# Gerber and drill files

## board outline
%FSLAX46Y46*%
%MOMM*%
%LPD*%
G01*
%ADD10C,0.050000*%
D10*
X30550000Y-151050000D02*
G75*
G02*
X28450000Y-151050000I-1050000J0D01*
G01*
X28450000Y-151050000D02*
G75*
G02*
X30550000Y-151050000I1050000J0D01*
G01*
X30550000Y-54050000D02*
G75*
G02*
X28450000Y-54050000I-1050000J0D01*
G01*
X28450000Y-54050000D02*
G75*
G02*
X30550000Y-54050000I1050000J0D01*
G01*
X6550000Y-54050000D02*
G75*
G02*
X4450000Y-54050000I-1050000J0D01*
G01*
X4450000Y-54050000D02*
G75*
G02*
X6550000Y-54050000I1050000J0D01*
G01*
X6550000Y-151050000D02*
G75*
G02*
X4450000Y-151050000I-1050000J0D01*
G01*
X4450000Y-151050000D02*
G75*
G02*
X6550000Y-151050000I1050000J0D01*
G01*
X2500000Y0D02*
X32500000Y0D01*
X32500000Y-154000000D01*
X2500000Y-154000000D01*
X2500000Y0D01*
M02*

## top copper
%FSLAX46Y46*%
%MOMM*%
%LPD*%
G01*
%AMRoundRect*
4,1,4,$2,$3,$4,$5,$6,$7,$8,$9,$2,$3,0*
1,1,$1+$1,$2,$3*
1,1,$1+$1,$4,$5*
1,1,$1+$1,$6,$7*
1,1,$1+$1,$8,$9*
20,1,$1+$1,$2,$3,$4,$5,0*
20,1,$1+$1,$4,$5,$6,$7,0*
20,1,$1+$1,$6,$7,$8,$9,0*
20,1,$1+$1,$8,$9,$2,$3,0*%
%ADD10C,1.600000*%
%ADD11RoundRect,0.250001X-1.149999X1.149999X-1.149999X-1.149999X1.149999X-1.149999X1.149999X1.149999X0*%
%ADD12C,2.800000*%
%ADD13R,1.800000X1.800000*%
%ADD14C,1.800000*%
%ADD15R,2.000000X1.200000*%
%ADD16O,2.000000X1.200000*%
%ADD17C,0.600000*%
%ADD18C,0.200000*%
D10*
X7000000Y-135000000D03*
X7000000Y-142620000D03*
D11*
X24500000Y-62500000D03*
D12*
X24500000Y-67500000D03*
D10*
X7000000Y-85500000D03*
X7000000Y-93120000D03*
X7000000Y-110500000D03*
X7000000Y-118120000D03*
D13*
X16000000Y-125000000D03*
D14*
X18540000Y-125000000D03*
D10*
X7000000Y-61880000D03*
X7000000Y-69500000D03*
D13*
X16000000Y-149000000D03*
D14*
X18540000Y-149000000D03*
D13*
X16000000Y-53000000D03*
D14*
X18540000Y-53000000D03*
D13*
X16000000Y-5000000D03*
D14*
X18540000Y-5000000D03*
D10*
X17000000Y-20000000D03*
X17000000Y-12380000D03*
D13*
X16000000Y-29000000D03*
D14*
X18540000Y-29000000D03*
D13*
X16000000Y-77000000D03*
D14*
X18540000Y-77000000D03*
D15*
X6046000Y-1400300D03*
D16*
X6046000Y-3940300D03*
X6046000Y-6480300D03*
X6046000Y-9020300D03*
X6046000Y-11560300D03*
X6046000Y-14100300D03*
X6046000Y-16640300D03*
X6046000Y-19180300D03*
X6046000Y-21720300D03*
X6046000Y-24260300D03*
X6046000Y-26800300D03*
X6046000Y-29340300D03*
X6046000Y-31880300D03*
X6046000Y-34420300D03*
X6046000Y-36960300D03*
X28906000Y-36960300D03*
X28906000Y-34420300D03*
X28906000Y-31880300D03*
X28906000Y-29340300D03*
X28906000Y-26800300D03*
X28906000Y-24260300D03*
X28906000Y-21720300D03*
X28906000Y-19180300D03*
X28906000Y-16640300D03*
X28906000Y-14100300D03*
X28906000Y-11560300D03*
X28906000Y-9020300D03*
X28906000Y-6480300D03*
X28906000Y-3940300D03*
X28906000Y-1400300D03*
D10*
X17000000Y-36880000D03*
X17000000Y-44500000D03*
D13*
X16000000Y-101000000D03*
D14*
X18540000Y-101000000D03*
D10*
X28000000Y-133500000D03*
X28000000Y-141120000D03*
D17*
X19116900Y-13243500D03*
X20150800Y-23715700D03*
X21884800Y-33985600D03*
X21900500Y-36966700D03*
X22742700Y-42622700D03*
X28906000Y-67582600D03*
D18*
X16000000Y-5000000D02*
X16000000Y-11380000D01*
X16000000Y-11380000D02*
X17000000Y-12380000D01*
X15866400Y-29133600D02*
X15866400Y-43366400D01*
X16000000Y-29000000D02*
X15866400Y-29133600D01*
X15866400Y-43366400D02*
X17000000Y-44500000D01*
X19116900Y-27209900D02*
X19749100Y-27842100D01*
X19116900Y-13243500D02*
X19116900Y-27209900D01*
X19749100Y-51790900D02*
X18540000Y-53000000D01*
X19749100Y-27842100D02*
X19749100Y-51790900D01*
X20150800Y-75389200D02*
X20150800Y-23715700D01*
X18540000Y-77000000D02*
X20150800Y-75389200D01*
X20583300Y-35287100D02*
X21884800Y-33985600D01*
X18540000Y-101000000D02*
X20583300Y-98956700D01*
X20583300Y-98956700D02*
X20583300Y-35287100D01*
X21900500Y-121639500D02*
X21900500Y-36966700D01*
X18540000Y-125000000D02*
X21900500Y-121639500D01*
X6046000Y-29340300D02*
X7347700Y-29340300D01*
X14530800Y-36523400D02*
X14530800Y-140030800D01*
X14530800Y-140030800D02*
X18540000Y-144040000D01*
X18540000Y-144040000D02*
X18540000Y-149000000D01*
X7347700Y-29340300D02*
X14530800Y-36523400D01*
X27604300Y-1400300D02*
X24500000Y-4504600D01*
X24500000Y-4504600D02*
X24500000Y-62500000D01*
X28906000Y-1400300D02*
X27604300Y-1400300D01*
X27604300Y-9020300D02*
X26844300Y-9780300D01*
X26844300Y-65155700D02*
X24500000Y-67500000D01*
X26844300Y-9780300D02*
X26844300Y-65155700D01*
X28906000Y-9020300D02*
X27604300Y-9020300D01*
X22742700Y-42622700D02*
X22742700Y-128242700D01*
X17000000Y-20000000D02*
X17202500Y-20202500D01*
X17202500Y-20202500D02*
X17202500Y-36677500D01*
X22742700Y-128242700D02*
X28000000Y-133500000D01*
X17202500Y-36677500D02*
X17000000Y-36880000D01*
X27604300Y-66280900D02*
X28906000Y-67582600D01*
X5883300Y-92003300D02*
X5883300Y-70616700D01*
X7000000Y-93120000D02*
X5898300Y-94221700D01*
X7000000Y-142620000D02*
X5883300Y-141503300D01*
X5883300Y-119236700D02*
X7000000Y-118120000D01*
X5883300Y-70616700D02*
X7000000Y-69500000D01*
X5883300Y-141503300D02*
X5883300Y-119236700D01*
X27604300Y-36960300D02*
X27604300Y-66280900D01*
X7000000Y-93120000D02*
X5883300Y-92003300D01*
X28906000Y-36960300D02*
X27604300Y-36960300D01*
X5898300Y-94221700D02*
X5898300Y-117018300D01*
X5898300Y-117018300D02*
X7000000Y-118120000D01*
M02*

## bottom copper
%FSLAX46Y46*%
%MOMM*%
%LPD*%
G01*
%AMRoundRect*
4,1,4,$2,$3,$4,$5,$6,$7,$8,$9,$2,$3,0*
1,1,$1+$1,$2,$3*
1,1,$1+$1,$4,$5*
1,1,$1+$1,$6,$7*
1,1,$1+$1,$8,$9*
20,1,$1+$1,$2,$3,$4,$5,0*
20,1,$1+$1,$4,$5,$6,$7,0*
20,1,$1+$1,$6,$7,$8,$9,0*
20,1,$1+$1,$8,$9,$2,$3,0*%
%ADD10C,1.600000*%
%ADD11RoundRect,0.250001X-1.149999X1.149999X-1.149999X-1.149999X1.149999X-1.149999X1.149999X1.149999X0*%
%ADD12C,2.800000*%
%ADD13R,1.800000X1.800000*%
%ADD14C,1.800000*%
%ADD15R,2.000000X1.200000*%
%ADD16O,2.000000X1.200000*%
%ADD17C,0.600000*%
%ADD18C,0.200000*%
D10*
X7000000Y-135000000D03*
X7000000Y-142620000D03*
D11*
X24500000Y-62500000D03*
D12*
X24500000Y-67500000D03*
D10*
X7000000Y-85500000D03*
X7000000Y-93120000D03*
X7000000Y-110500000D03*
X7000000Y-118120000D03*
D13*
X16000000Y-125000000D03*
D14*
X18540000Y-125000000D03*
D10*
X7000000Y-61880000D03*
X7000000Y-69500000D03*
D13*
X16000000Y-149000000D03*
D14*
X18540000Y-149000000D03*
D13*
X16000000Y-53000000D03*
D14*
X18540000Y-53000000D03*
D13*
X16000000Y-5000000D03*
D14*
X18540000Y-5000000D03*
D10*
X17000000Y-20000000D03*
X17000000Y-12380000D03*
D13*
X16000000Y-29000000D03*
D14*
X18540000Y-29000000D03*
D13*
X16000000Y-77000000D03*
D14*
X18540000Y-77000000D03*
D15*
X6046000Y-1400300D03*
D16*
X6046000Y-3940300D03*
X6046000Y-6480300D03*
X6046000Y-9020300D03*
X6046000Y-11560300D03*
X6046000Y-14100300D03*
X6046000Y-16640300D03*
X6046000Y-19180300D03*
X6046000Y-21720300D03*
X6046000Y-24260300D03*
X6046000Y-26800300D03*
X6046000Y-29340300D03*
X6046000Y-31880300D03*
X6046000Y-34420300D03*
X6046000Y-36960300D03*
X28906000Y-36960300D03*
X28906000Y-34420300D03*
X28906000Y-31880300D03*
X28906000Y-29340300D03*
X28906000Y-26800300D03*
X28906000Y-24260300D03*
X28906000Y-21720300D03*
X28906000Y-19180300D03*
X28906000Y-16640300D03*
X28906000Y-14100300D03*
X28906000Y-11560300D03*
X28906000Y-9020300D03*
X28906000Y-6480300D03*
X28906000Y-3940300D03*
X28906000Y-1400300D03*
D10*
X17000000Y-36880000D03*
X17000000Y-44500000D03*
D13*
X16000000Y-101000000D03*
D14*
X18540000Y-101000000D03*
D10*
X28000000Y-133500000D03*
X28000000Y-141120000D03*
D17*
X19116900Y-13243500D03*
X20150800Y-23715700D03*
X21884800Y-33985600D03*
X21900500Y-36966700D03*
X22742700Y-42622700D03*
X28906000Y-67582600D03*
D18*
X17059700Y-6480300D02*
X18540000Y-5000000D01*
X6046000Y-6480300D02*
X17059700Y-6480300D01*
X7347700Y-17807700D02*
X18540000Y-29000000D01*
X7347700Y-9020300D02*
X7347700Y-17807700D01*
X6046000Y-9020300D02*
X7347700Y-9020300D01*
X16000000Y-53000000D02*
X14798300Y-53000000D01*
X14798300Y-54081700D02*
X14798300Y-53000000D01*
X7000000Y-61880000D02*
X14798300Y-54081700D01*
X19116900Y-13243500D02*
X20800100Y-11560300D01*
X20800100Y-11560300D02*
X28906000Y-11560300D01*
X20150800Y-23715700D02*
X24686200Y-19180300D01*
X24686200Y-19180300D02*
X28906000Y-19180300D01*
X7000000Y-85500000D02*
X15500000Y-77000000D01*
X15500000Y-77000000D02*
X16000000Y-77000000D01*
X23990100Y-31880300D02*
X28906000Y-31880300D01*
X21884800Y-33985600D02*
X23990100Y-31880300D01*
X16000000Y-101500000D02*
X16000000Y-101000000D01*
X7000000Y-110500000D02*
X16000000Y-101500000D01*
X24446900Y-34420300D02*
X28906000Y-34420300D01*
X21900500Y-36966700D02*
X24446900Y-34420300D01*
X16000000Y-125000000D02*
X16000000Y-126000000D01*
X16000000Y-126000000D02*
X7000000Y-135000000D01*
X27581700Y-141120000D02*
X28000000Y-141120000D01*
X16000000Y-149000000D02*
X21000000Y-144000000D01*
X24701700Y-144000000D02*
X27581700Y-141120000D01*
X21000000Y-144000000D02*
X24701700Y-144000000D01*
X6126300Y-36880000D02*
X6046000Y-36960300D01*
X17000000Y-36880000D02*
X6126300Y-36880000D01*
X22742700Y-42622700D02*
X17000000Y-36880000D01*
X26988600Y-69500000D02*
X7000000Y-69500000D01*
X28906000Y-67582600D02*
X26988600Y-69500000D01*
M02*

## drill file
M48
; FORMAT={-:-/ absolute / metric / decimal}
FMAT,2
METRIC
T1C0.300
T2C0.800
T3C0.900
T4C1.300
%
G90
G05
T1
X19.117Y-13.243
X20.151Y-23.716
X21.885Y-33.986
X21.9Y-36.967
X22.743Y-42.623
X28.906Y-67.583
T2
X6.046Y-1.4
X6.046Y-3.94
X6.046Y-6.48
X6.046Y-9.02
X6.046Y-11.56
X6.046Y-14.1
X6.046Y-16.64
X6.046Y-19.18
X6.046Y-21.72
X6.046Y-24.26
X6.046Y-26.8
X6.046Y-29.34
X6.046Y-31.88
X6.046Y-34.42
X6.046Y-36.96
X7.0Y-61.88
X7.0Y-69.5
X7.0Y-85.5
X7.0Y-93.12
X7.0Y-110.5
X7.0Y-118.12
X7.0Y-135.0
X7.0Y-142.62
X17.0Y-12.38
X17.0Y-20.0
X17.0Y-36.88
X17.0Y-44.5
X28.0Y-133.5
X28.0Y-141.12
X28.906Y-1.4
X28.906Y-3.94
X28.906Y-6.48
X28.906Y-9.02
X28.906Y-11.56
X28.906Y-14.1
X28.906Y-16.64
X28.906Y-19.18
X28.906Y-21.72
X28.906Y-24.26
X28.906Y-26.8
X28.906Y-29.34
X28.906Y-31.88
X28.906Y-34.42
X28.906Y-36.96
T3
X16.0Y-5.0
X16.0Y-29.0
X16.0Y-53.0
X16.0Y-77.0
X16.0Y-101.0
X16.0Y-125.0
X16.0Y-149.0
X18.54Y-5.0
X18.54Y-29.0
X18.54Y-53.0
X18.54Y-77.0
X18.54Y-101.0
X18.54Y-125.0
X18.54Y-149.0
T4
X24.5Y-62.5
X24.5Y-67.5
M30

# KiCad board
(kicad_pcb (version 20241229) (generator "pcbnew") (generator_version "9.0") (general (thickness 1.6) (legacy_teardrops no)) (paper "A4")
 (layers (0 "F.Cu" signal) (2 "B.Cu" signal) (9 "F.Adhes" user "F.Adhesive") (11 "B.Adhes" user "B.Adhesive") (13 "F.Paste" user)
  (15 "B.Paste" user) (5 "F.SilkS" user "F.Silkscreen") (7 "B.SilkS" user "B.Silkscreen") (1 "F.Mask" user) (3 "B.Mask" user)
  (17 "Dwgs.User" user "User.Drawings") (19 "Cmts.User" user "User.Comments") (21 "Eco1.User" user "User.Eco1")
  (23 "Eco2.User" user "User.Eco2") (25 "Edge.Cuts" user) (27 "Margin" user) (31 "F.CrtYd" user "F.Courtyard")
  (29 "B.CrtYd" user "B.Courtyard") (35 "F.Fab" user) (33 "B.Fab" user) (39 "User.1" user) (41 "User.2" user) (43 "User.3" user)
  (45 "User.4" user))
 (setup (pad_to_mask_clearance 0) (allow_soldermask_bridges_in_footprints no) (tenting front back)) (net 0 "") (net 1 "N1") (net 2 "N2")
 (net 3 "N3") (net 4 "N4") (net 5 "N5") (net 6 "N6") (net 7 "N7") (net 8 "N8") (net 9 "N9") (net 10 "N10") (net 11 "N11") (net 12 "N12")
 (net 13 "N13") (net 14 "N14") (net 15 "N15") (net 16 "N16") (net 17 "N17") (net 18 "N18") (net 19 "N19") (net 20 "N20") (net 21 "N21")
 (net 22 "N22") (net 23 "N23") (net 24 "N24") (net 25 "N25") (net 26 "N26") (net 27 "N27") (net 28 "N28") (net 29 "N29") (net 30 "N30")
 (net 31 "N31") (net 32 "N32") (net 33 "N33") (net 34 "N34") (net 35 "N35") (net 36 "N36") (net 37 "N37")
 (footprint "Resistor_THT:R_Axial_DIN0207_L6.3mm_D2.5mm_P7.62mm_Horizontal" (layer "F.Cu") (at 7 135 -90)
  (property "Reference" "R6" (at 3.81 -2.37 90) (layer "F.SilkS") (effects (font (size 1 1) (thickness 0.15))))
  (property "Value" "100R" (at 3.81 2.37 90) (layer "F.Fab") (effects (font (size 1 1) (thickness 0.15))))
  (pad "1" thru_hole circle (at 0 0 270) (size 1.6 1.6) (drill 0.8) (layers "*.Cu" "*.Mask") (remove_unused_layers no) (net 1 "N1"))
  (pad "2" thru_hole circle (at 7.62 0 270) (size 1.6 1.6) (drill 0.8) (layers "*.Cu" "*.Mask") (remove_unused_layers no) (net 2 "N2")))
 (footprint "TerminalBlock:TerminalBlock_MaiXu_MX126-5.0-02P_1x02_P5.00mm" (layer "F.Cu") (at 24.5 62.5 -90)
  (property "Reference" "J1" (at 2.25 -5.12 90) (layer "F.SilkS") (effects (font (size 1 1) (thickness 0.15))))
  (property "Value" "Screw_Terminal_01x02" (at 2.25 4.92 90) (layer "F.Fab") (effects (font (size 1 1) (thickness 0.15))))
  (pad "1" thru_hole roundrect (at 0 0 270) (size 2.8 2.8) (drill 1.3) (layers "*.Cu" "*.Mask") (remove_unused_layers no)
   (roundrect_rratio 0.089286) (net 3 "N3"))
  (pad "2" thru_hole circle (at 5 0 270) (size 2.8 2.8) (drill 1.3) (layers "*.Cu" "*.Mask") (remove_unused_layers no) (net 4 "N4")))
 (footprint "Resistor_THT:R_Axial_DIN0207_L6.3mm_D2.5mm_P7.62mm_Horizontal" (layer "F.Cu") (at 7 85.5 -90)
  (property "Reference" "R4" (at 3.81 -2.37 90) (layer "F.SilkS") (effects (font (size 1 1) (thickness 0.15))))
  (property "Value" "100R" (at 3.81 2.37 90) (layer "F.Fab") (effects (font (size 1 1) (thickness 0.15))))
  (pad "1" thru_hole circle (at 0 0 270) (size 1.6 1.6) (drill 0.8) (layers "*.Cu" "*.Mask") (remove_unused_layers no) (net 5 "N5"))
  (pad "2" thru_hole circle (at 7.62 0 270) (size 1.6 1.6) (drill 0.8) (layers "*.Cu" "*.Mask") (remove_unused_layers no) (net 2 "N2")))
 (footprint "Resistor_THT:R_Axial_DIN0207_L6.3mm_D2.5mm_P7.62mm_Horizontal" (layer "F.Cu") (at 7 110.5 -90)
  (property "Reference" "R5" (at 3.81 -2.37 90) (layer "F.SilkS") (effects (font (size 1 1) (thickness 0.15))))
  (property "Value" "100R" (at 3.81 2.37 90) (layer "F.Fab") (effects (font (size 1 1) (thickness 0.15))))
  (pad "1" thru_hole circle (at 0 0 270) (size 1.6 1.6) (drill 0.8) (layers "*.Cu" "*.Mask") (remove_unused_layers no) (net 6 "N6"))
  (pad "2" thru_hole circle (at 7.62 0 270) (size 1.6 1.6) (drill 0.8) (layers "*.Cu" "*.Mask") (remove_unused_layers no) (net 2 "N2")))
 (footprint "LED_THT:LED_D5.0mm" (layer "F.Cu") (at 16 125)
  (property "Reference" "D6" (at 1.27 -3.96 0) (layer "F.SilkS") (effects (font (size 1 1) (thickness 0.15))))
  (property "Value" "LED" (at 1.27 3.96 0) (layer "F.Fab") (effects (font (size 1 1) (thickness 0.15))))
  (pad "1" thru_hole rect (at 0 0) (size 1.8 1.8) (drill 0.9) (layers "*.Cu" "*.Mask") (remove_unused_layers no) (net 1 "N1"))
  (pad "2" thru_hole circle (at 2.54 0) (size 1.8 1.8) (drill 0.9) (layers "*.Cu" "*.Mask") (remove_unused_layers no) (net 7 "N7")))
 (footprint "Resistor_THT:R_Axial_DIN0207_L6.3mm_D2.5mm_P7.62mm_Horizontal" (layer "F.Cu") (at 7 61.88 -90)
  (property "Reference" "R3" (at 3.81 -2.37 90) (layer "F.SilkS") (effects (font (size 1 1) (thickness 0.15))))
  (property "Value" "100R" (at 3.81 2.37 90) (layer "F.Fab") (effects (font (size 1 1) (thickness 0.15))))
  (pad "1" thru_hole circle (at 0 0 270) (size 1.6 1.6) (drill 0.8) (layers "*.Cu" "*.Mask") (remove_unused_layers no) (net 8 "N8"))
  (pad "2" thru_hole circle (at 7.62 0 270) (size 1.6 1.6) (drill 0.8) (layers "*.Cu" "*.Mask") (remove_unused_layers no) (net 2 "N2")))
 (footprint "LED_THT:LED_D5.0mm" (layer "F.Cu") (at 16 149)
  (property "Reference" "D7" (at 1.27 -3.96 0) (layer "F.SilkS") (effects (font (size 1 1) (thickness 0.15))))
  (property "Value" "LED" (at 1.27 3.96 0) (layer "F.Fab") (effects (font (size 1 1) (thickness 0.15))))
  (pad "1" thru_hole rect (at 0 0) (size 1.8 1.8) (drill 0.9) (layers "*.Cu" "*.Mask") (remove_unused_layers no) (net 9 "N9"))
  (pad "2" thru_hole circle (at 2.54 0) (size 1.8 1.8) (drill 0.9) (layers "*.Cu" "*.Mask") (remove_unused_layers no) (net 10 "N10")))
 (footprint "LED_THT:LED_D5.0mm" (layer "F.Cu") (at 16 53)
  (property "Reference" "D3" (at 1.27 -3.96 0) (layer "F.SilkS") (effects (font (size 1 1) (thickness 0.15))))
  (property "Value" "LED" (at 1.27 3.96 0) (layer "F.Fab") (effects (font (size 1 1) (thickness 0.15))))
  (pad "1" thru_hole rect (at 0 0) (size 1.8 1.8) (drill 0.9) (layers "*.Cu" "*.Mask") (remove_unused_layers no) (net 8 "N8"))
  (pad "2" thru_hole circle (at 2.54 0) (size 1.8 1.8) (drill 0.9) (layers "*.Cu" "*.Mask") (remove_unused_layers no) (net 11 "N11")))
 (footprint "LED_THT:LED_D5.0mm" (layer "F.Cu") (at 16 5)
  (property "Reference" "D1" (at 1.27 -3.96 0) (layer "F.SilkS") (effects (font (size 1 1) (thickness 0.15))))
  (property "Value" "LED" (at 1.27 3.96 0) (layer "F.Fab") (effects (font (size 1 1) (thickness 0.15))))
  (pad "1" thru_hole rect (at 0 0) (size 1.8 1.8) (drill 0.9) (layers "*.Cu" "*.Mask") (remove_unused_layers no) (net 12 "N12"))
  (pad "2" thru_hole circle (at 2.54 0) (size 1.8 1.8) (drill 0.9) (layers "*.Cu" "*.Mask") (remove_unused_layers no) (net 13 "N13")))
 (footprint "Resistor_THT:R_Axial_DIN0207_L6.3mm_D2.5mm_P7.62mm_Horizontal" (layer "F.Cu") (at 17 20 90)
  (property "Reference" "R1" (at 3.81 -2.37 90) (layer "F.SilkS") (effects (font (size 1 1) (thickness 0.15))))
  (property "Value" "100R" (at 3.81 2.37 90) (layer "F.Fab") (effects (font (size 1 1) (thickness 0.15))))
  (pad "1" thru_hole circle (at 0 0 90) (size 1.6 1.6) (drill 0.8) (layers "*.Cu" "*.Mask") (remove_unused_layers no) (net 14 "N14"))
  (pad "2" thru_hole circle (at 7.62 0 90) (size 1.6 1.6) (drill 0.8) (layers "*.Cu" "*.Mask") (remove_unused_layers no) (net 12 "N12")))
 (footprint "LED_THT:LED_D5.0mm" (layer "F.Cu") (at 16 29)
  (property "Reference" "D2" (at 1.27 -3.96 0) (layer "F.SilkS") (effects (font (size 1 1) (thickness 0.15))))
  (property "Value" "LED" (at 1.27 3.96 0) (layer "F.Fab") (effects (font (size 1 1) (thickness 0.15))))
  (pad "1" thru_hole rect (at 0 0) (size 1.8 1.8) (drill 0.9) (layers "*.Cu" "*.Mask") (remove_unused_layers no) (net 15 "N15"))
  (pad "2" thru_hole circle (at 2.54 0) (size 1.8 1.8) (drill 0.9) (layers "*.Cu" "*.Mask") (remove_unused_layers no) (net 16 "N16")))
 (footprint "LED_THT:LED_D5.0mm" (layer "F.Cu") (at 16 77)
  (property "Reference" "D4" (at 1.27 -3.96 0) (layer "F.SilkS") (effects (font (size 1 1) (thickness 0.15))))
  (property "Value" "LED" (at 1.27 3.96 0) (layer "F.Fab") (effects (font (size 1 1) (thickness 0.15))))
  (pad "1" thru_hole rect (at 0 0) (size 1.8 1.8) (drill 0.9) (layers "*.Cu" "*.Mask") (remove_unused_layers no) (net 5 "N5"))
  (pad "2" thru_hole circle (at 2.54 0) (size 1.8 1.8) (drill 0.9) (layers "*.Cu" "*.Mask") (remove_unused_layers no) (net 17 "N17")))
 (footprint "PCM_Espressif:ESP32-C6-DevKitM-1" (layer "F.Cu") (at 6.046 1.4003)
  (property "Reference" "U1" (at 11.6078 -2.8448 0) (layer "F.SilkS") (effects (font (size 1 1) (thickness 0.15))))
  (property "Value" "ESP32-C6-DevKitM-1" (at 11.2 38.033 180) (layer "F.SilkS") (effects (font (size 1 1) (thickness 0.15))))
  (pad "1" thru_hole rect (at 0 0 270) (size 1.2 2) (drill 0.8) (layers "*.Cu" "*.Mask") (remove_unused_layers no) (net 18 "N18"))
  (pad "2" thru_hole oval (at 0 2.54 270) (size 1.2 2) (drill 0.8) (layers "*.Cu" "*.Mask") (remove_unused_layers no) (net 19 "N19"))
  (pad "3" thru_hole oval (at 0 5.08 270) (size 1.2 2) (drill 0.8) (layers "*.Cu" "*.Mask") (remove_unused_layers no) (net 13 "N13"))
  (pad "4" thru_hole oval (at 0 7.62 270) (size 1.2 2) (drill 0.8) (layers "*.Cu" "*.Mask") (remove_unused_layers no) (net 16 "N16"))
  (pad "5" thru_hole oval (at 0 10.16 270) (size 1.2 2) (drill 0.8) (layers "*.Cu" "*.Mask") (remove_unused_layers no) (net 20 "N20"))
  (pad "6" thru_hole oval (at 0 12.7 270) (size 1.2 2) (drill 0.8) (layers "*.Cu" "*.Mask") (remove_unused_layers no) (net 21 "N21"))
  (pad "7" thru_hole oval (at 0 15.24 270) (size 1.2 2) (drill 0.8) (layers "*.Cu" "*.Mask") (remove_unused_layers no) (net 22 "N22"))
  (pad "8" thru_hole oval (at 0 17.78 270) (size 1.2 2) (drill 0.8) (layers "*.Cu" "*.Mask") (remove_unused_layers no) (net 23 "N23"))
  (pad "9" thru_hole oval (at 0 20.32 270) (size 1.2 2) (drill 0.8) (layers "*.Cu" "*.Mask") (remove_unused_layers no) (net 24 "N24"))
  (pad "10" thru_hole oval (at 0 22.86 270) (size 1.2 2) (drill 0.8) (layers "*.Cu" "*.Mask") (remove_unused_layers no) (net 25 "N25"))
  (pad "11" thru_hole oval (at 0 25.4 270) (size 1.2 2) (drill 0.8) (layers "*.Cu" "*.Mask") (remove_unused_layers no) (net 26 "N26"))
  (pad "12" thru_hole oval (at 0 27.94 270) (size 1.2 2) (drill 0.8) (layers "*.Cu" "*.Mask") (remove_unused_layers no) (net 10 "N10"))
  (pad "13" thru_hole oval (at 0 30.48 270) (size 1.2 2) (drill 0.8) (layers "*.Cu" "*.Mask") (remove_unused_layers no) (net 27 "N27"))
  (pad "14" thru_hole oval (at 0 33.02 270) (size 1.2 2) (drill 0.8) (layers "*.Cu" "*.Mask") (remove_unused_layers no) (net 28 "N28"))
  (pad "15" thru_hole oval (at 0 35.56 270) (size 1.2 2) (drill 0.8) (layers "*.Cu" "*.Mask") (remove_unused_layers no) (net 14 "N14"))
  (pad "16" thru_hole oval (at 22.86 35.56 270) (size 1.2 2) (drill 0.8) (layers "*.Cu" "*.Mask") (remove_unused_layers no) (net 2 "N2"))
  (pad "17" thru_hole oval (at 22.86 33.02 270) (size 1.2 2) (drill 0.8) (layers "*.Cu" "*.Mask") (remove_unused_layers no) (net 7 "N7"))
  (pad "18" thru_hole oval (at 22.86 30.48 270) (size 1.2 2) (drill 0.8) (layers "*.Cu" "*.Mask") (remove_unused_layers no) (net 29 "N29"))
  (pad "19" thru_hole oval (at 22.86 27.94 270) (size 1.2 2) (drill 0.8) (layers "*.Cu" "*.Mask") (remove_unused_layers no) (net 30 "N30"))
  (pad "20" thru_hole oval (at 22.86 25.4 270) (size 1.2 2) (drill 0.8) (layers "*.Cu" "*.Mask") (remove_unused_layers no) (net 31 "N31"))
  (pad "21" thru_hole oval (at 22.86 22.86 270) (size 1.2 2) (drill 0.8) (layers "*.Cu" "*.Mask") (remove_unused_layers no) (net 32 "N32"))
  (pad "22" thru_hole oval (at 22.86 20.32 270) (size 1.2 2) (drill 0.8) (layers "*.Cu" "*.Mask") (remove_unused_layers no) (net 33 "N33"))
  (pad "23" thru_hole oval (at 22.86 17.78 270) (size 1.2 2) (drill 0.8) (layers "*.Cu" "*.Mask") (remove_unused_layers no) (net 17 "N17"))
  (pad "24" thru_hole oval (at 22.86 15.24 270) (size 1.2 2) (drill 0.8) (layers "*.Cu" "*.Mask") (remove_unused_layers no) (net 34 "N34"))
  (pad "25" thru_hole oval (at 22.86 12.7 270) (size 1.2 2) (drill 0.8) (layers "*.Cu" "*.Mask") (remove_unused_layers no) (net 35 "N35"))
  (pad "26" thru_hole oval (at 22.86 10.16 270) (size 1.2 2) (drill 0.8) (layers "*.Cu" "*.Mask") (remove_unused_layers no) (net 11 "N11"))
  (pad "27" thru_hole oval (at 22.86 7.62 270) (size 1.2 2) (drill 0.8) (layers "*.Cu" "*.Mask") (remove_unused_layers no) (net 4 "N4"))
  (pad "28" thru_hole oval (at 22.86 5.08 270) (size 1.2 2) (drill 0.8) (layers "*.Cu" "*.Mask") (remove_unused_layers no) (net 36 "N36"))
  (pad "29" thru_hole oval (at 22.86 2.54 270) (size 1.2 2) (drill 0.8) (layers "*.Cu" "*.Mask") (remove_unused_layers no) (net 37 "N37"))
  (pad "30" thru_hole oval (at 22.86 0 270) (size 1.2 2) (drill 0.8) (layers "*.Cu" "*.Mask") (remove_unused_layers no) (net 3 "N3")))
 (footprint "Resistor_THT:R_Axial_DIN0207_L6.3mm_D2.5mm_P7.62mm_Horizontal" (layer "F.Cu") (at 17 36.88 -90)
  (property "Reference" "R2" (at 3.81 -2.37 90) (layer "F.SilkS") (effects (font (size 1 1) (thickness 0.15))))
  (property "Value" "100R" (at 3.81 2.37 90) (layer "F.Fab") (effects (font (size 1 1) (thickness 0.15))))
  (pad "1" thru_hole circle (at 0 0 270) (size 1.6 1.6) (drill 0.8) (layers "*.Cu" "*.Mask") (remove_unused_layers no) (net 14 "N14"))
  (pad "2" thru_hole circle (at 7.62 0 270) (size 1.6 1.6) (drill 0.8) (layers "*.Cu" "*.Mask") (remove_unused_layers no) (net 15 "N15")))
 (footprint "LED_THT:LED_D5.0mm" (layer "F.Cu") (at 16 101)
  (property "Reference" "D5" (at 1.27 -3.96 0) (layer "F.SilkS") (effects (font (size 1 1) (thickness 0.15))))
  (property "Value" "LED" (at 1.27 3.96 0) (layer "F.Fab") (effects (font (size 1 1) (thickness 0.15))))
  (pad "1" thru_hole rect (at 0 0) (size 1.8 1.8) (drill 0.9) (layers "*.Cu" "*.Mask") (remove_unused_layers no) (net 6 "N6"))
  (pad "2" thru_hole circle (at 2.54 0) (size 1.8 1.8) (drill 0.9) (layers "*.Cu" "*.Mask") (remove_unused_layers no) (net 29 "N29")))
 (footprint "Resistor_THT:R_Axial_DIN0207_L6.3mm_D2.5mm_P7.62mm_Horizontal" (layer "F.Cu") (at 28 133.5 -90)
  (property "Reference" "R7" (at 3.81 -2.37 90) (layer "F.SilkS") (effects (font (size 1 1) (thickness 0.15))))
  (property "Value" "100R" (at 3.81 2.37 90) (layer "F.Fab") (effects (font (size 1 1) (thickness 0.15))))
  (pad "1" thru_hole circle (at 0 0 270) (size 1.6 1.6) (drill 0.8) (layers "*.Cu" "*.Mask") (remove_unused_layers no) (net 14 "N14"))
  (pad "2" thru_hole circle (at 7.62 0 270) (size 1.6 1.6) (drill 0.8) (layers "*.Cu" "*.Mask") (remove_unused_layers no) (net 9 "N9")))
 (gr_circle (center 29.5 151.05) (end 30.55 151.05) (stroke (width 0.05) (type solid)) (fill no) (layer "Edge.Cuts"))
 (gr_circle (center 29.5 54.05) (end 30.55 54.05) (stroke (width 0.05) (type solid)) (fill no) (layer "Edge.Cuts"))
 (gr_circle (center 5.5 54.05) (end 6.55 54.05) (stroke (width 0.05) (type solid)) (fill no) (layer "Edge.Cuts"))
 (gr_circle (center 5.5 151.05) (end 6.55 151.05) (stroke (width 0.05) (type solid)) (fill no) (layer "Edge.Cuts"))
 (gr_rect (start 2.5 0) (end 32.5 154) (stroke (width 0.05) (type solid)) (fill no) (layer "Edge.Cuts"))
 (segment (start 16 5) (end 16 11.38) (width 0.2) (layer "F.Cu") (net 12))
 (segment (start 16 11.38) (end 17 12.38) (width 0.2) (layer "F.Cu") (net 12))
 (segment (start 17.0597 6.4803) (end 18.54 5) (width 0.2) (layer "B.Cu") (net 13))
 (segment (start 6.046 6.4803) (end 17.0597 6.4803) (width 0.2) (layer "B.Cu") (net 13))
 (segment (start 15.8664 29.1336) (end 15.8664 43.3664) (width 0.2) (layer "F.Cu") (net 15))
 (segment (start 16 29) (end 15.8664 29.1336) (width 0.2) (layer "F.Cu") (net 15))
 (segment (start 15.8664 43.3664) (end 17 44.5) (width 0.2) (layer "F.Cu") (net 15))
 (segment (start 7.3477 17.8077) (end 18.54 29) (width 0.2) (layer "B.Cu") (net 16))
 (segment (start 7.3477 9.0203) (end 7.3477 17.8077) (width 0.2) (layer "B.Cu") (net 16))
 (segment (start 6.046 9.0203) (end 7.3477 9.0203) (width 0.2) (layer "B.Cu") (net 16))
 (segment (start 16 53) (end 14.7983 53) (width 0.2) (layer "B.Cu") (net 8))
 (segment (start 14.7983 54.0817) (end 14.7983 53) (width 0.2) (layer "B.Cu") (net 8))
 (segment (start 7 61.88) (end 14.7983 54.0817) (width 0.2) (layer "B.Cu") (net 8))
 (segment (start 19.1169 27.2099) (end 19.7491 27.8421) (width 0.2) (layer "F.Cu") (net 11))
 (segment (start 19.1169 13.2435) (end 19.1169 27.2099) (width 0.2) (layer "F.Cu") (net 11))
 (segment (start 19.7491 51.7909) (end 18.54 53) (width 0.2) (layer "F.Cu") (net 11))
 (segment (start 19.7491 27.8421) (end 19.7491 51.7909) (width 0.2) (layer "F.Cu") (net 11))
 (via (at 19.1169 13.2435) (size 0.6) (drill 0.3) (layers "F.Cu" "B.Cu") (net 11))
 (segment (start 19.1169 13.2435) (end 20.8001 11.5603) (width 0.2) (layer "B.Cu") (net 11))
 (segment (start 20.8001 11.5603) (end 28.906 11.5603) (width 0.2) (layer "B.Cu") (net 11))
 (segment (start 20.1508 75.3892) (end 20.1508 23.7157) (width 0.2) (layer "F.Cu") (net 17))
 (segment (start 18.54 77) (end 20.1508 75.3892) (width 0.2) (layer "F.Cu") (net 17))
 (via (at 20.1508 23.7157) (size 0.6) (drill 0.3) (layers "F.Cu" "B.Cu") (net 17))
 (segment (start 20.1508 23.7157) (end 24.6862 19.1803) (width 0.2) (layer "B.Cu") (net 17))
 (segment (start 24.6862 19.1803) (end 28.906 19.1803) (width 0.2) (layer "B.Cu") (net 17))
 (segment (start 7 85.5) (end 15.5 77) (width 0.2) (layer "B.Cu") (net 5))
 (segment (start 15.5 77) (end 16 77) (width 0.2) (layer "B.Cu") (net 5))
 (segment (start 20.5833 35.2871) (end 21.8848 33.9856) (width 0.2) (layer "F.Cu") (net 29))
 (segment (start 18.54 101) (end 20.5833 98.9567) (width 0.2) (layer "F.Cu") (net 29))
 (segment (start 20.5833 98.9567) (end 20.5833 35.2871) (width 0.2) (layer "F.Cu") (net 29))
 (via (at 21.8848 33.9856) (size 0.6) (drill 0.3) (layers "F.Cu" "B.Cu") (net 29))
 (segment (start 23.9901 31.8803) (end 28.906 31.8803) (width 0.2) (layer "B.Cu") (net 29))
 (segment (start 21.8848 33.9856) (end 23.9901 31.8803) (width 0.2) (layer "B.Cu") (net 29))
 (segment (start 16 101.5) (end 16 101) (width 0.2) (layer "B.Cu") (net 6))
 (segment (start 7 110.5) (end 16 101.5) (width 0.2) (layer "B.Cu") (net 6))
 (segment (start 21.9005 121.6395) (end 21.9005 36.9667) (width 0.2) (layer "F.Cu") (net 7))
 (segment (start 18.54 125) (end 21.9005 121.6395) (width 0.2) (layer "F.Cu") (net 7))
 (via (at 21.9005 36.9667) (size 0.6) (drill 0.3) (layers "F.Cu" "B.Cu") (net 7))
 (segment (start 24.4469 34.4203) (end 28.906 34.4203) (width 0.2) (layer "B.Cu") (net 7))
 (segment (start 21.9005 36.9667) (end 24.4469 34.4203) (width 0.2) (layer "B.Cu") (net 7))
 (segment (start 16 125) (end 16 126) (width 0.2) (layer "B.Cu") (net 1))
 (segment (start 16 126) (end 7 135) (width 0.2) (layer "B.Cu") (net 1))
 (segment (start 27.5817 141.12) (end 28 141.12) (width 0.2) (layer "B.Cu") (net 9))
 (segment (start 16 149) (end 21 144) (width 0.2) (layer "B.Cu") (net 9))
 (segment (start 24.7017 144) (end 27.5817 141.12) (width 0.2) (layer "B.Cu") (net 9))
 (segment (start 21 144) (end 24.7017 144) (width 0.2) (layer "B.Cu") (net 9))
 (segment (start 6.046 29.3403) (end 7.3477 29.3403) (width 0.2) (layer "F.Cu") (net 10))
 (segment (start 14.5308 36.5234) (end 14.5308 140.0308) (width 0.2) (layer "F.Cu") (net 10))
 (segment (start 14.5308 140.0308) (end 18.54 144.04) (width 0.2) (layer "F.Cu") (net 10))
 (segment (start 18.54 144.04) (end 18.54 149) (width 0.2) (layer "F.Cu") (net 10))
 (segment (start 7.3477 29.3403) (end 14.5308 36.5234) (width 0.2) (layer "F.Cu") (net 10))
 (segment (start 27.6043 1.4003) (end 24.5 4.5046) (width 0.2) (layer "F.Cu") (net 3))
 (segment (start 24.5 4.5046) (end 24.5 62.5) (width 0.2) (layer "F.Cu") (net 3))
 (segment (start 28.906 1.4003) (end 27.6043 1.4003) (width 0.2) (layer "F.Cu") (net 3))
 (segment (start 27.6043 9.0203) (end 26.8443 9.7803) (width 0.2) (layer "F.Cu") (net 4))
 (segment (start 26.8443 65.1557) (end 24.5 67.5) (width 0.2) (layer "F.Cu") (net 4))
 (segment (start 26.8443 9.7803) (end 26.8443 65.1557) (width 0.2) (layer "F.Cu") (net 4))
 (segment (start 28.906 9.0203) (end 27.6043 9.0203) (width 0.2) (layer "F.Cu") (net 4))
 (segment (start 22.7427 42.6227) (end 22.7427 128.2427) (width 0.2) (layer "F.Cu") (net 14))
 (segment (start 17 20) (end 17.2025 20.2025) (width 0.2) (layer "F.Cu") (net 14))
 (segment (start 17.2025 20.2025) (end 17.2025 36.6775) (width 0.2) (layer "F.Cu") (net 14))
 (segment (start 22.7427 128.2427) (end 28 133.5) (width 0.2) (layer "F.Cu") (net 14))
 (segment (start 17.2025 36.6775) (end 17 36.88) (width 0.2) (layer "F.Cu") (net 14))
 (via (at 22.7427 42.6227) (size 0.6) (drill 0.3) (layers "F.Cu" "B.Cu") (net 14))
 (segment (start 6.1263 36.88) (end 6.046 36.9603) (width 0.2) (layer "B.Cu") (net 14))
 (segment (start 17 36.88) (end 6.1263 36.88) (width 0.2) (layer "B.Cu") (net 14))
 (segment (start 22.7427 42.6227) (end 17 36.88) (width 0.2) (layer "B.Cu") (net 14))
 (segment (start 27.6043 66.2809) (end 28.906 67.5826) (width 0.2) (layer "F.Cu") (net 2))
 (segment (start 5.8833 92.0033) (end 5.8833 70.6167) (width 0.2) (layer "F.Cu") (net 2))
 (segment (start 7 93.12) (end 5.8983 94.2217) (width 0.2) (layer "F.Cu") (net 2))
 (segment (start 7 142.62) (end 5.8833 141.5033) (width 0.2) (layer "F.Cu") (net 2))
 (segment (start 5.8833 119.2367) (end 7 118.12) (width 0.2) (layer "F.Cu") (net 2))
 (segment (start 5.8833 70.6167) (end 7 69.5) (width 0.2) (layer "F.Cu") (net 2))
 (segment (start 5.8833 141.5033) (end 5.8833 119.2367) (width 0.2) (layer "F.Cu") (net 2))
 (segment (start 27.6043 36.9603) (end 27.6043 66.2809) (width 0.2) (layer "F.Cu") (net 2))
 (segment (start 7 93.12) (end 5.8833 92.0033) (width 0.2) (layer "F.Cu") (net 2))
 (segment (start 28.906 36.9603) (end 27.6043 36.9603) (width 0.2) (layer "F.Cu") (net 2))
 (segment (start 5.8983 94.2217) (end 5.8983 117.0183) (width 0.2) (layer "F.Cu") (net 2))
 (segment (start 5.8983 117.0183) (end 7 118.12) (width 0.2) (layer "F.Cu") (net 2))
 (via (at 28.906 67.5826) (size 0.6) (drill 0.3) (layers "F.Cu" "B.Cu") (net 2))
 (segment (start 26.9886 69.5) (end 7 69.5) (width 0.2) (layer "B.Cu") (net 2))
 (segment (start 28.906 67.5826) (end 26.9886 69.5) (width 0.2) (layer "B.Cu") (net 2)))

